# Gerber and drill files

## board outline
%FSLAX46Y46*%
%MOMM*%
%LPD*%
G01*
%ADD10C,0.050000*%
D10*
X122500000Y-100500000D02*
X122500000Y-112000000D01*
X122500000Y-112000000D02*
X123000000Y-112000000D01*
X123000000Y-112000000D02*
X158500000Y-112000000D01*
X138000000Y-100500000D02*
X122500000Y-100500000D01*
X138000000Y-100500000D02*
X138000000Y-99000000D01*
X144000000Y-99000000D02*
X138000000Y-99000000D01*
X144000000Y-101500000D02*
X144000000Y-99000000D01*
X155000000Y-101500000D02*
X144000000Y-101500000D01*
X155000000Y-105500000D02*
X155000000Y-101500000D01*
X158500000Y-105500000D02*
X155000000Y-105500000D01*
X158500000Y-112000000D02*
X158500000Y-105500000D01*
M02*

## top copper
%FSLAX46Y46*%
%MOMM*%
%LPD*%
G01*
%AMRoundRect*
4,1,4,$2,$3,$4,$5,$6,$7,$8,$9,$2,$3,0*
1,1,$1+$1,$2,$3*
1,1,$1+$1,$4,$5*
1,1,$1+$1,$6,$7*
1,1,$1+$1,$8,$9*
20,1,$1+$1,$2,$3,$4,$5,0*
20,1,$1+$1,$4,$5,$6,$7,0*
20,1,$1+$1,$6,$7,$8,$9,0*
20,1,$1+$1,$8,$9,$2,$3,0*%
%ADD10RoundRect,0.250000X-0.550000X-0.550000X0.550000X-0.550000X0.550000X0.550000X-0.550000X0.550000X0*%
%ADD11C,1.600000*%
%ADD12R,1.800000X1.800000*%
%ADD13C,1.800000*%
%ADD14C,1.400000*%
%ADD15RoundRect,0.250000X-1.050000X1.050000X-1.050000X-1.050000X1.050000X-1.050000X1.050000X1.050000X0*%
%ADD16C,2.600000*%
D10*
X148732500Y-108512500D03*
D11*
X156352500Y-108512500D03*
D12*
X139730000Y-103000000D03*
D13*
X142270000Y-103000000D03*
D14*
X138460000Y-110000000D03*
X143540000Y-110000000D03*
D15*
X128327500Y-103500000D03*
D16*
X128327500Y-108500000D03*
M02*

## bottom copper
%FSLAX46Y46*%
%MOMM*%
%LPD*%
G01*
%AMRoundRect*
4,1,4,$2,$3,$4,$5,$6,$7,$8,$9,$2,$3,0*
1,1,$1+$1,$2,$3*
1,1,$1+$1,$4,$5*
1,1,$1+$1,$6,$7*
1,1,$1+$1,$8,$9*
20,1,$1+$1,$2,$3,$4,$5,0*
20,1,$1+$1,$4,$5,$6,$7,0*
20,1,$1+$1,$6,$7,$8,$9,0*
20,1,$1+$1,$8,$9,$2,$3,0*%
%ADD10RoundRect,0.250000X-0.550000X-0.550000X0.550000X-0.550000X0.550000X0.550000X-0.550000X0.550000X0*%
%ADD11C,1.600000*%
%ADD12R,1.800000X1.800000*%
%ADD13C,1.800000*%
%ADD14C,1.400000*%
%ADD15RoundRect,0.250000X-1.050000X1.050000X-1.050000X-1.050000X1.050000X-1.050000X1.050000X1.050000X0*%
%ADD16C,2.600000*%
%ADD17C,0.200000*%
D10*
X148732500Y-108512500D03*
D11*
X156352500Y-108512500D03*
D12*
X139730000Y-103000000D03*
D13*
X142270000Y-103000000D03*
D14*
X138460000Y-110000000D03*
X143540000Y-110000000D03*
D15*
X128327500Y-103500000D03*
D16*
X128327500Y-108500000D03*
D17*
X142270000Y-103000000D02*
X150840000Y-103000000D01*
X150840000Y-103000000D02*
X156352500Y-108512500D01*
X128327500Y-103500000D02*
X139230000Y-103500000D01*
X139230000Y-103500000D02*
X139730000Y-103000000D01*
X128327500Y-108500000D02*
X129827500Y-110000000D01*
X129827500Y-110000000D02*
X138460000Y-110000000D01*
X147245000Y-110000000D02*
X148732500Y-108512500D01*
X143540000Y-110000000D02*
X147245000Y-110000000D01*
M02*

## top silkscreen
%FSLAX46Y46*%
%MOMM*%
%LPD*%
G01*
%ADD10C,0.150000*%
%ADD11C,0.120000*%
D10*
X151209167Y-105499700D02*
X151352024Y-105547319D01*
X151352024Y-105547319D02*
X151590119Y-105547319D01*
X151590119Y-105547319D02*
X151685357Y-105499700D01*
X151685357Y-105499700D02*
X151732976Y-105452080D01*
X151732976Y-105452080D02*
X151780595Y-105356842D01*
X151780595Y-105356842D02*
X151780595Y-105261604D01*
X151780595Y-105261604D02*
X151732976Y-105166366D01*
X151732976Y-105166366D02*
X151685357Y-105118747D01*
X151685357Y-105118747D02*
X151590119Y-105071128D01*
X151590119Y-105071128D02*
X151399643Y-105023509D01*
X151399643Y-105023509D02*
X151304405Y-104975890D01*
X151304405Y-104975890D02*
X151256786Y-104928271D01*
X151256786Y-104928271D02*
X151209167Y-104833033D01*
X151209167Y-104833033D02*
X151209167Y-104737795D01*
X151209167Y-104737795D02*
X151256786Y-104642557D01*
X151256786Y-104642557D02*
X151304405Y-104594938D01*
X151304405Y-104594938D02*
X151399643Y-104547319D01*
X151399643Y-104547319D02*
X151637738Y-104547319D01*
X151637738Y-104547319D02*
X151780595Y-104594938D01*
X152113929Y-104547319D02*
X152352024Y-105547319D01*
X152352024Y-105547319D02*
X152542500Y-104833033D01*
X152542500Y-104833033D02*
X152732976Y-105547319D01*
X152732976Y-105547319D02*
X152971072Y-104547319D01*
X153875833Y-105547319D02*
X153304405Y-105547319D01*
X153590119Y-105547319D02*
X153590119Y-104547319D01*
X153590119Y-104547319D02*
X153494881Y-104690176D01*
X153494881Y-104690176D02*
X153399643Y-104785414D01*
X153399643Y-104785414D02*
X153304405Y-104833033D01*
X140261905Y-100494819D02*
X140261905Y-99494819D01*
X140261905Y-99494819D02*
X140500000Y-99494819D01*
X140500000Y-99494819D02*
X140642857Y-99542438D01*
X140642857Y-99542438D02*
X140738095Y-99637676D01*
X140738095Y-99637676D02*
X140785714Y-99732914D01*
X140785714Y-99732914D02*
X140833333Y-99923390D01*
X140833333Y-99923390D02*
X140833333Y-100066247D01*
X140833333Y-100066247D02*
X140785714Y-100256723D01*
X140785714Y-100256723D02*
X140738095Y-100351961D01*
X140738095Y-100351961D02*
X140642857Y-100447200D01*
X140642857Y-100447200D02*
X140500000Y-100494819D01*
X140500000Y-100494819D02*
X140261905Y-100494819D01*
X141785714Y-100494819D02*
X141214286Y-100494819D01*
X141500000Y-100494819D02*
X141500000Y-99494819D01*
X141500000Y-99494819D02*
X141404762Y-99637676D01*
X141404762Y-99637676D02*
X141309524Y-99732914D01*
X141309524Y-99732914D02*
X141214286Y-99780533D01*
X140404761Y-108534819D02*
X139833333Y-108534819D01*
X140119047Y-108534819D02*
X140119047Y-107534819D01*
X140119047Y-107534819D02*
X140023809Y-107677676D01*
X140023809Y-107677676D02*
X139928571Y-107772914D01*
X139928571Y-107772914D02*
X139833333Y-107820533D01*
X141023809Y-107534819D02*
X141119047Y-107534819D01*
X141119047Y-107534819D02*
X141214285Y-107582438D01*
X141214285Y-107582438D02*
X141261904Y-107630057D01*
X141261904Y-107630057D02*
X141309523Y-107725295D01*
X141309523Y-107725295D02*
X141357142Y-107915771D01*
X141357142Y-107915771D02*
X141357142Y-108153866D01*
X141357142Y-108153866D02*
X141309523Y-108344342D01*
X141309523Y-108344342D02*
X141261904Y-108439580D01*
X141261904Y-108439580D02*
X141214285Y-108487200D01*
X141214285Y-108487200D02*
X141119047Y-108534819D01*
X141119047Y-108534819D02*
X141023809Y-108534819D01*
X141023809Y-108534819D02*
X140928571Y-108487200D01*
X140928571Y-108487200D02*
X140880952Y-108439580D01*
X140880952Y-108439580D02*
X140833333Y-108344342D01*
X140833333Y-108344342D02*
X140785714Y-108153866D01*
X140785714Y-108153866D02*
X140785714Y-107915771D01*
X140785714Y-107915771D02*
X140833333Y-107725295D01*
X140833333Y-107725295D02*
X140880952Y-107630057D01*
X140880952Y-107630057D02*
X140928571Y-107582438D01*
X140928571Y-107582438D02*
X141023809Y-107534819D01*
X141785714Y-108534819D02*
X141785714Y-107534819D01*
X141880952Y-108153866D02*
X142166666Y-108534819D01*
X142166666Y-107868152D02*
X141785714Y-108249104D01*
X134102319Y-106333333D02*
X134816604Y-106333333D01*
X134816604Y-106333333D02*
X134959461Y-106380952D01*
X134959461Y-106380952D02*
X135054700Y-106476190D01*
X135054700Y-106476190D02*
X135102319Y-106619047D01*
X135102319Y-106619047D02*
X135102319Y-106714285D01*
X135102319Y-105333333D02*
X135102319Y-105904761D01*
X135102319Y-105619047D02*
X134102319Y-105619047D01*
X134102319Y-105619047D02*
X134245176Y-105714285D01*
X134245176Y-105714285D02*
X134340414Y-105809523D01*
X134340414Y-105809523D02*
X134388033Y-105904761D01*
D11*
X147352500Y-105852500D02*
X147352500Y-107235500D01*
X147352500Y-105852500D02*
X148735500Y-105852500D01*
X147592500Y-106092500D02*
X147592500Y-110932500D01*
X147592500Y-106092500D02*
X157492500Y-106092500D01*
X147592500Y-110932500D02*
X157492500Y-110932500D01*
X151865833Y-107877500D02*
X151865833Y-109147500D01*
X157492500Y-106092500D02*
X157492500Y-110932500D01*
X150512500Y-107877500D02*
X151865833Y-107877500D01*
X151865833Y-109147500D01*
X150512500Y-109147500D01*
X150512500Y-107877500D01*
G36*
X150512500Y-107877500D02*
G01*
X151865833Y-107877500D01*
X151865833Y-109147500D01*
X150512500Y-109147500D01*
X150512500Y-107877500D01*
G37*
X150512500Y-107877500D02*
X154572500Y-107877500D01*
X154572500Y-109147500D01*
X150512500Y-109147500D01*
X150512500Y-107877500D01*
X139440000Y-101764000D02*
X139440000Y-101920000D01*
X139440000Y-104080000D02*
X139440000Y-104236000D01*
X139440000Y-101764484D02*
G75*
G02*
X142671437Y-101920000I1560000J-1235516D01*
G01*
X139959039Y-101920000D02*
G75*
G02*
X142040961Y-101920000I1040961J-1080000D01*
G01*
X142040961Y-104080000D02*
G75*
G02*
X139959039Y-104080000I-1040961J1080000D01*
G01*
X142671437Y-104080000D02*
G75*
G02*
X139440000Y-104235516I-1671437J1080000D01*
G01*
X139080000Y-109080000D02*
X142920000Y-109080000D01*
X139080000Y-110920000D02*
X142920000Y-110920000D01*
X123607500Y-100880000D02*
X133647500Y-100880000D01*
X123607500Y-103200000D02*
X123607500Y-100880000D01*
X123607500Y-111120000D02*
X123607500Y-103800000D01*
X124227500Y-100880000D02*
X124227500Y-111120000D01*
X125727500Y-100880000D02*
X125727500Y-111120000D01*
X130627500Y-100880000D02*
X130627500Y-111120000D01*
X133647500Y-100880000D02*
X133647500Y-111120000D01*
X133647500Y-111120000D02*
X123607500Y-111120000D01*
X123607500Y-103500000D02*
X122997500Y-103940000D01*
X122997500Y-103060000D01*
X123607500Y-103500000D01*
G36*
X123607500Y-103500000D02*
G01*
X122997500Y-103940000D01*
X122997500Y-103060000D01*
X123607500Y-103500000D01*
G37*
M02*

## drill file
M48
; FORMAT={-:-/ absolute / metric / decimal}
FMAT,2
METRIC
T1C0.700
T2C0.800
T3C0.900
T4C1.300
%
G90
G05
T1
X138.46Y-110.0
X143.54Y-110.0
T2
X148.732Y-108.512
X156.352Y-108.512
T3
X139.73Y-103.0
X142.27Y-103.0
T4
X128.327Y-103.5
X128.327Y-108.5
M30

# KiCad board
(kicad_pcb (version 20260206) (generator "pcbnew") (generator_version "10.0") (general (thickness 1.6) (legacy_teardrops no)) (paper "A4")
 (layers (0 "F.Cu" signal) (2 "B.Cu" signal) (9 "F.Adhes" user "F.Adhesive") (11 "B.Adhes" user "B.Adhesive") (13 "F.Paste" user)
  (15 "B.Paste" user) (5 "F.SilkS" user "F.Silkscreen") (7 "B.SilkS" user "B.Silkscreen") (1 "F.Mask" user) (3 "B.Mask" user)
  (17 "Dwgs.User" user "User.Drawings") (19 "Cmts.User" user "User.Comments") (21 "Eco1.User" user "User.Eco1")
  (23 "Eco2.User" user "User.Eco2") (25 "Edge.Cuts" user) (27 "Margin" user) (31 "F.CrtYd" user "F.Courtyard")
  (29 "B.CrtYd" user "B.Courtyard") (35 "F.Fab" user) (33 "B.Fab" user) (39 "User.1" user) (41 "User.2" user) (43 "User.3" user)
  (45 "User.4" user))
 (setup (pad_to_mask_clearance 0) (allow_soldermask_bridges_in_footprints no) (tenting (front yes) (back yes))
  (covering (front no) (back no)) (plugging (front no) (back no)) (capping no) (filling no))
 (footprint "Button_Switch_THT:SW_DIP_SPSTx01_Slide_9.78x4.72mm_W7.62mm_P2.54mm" (layer "F.Cu") (at 148.7325 108.5125)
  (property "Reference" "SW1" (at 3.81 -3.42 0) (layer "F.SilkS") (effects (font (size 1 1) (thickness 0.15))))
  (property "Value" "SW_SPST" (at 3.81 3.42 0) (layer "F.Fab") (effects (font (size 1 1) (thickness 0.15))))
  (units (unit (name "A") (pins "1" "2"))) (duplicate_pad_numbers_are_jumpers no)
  (fp_line (start -1.38 -2.66) (end -1.38 -1.277) (stroke (width 0.12) (type solid)) (layer "F.SilkS"))
  (fp_line (start -1.38 -2.66) (end 0.003 -2.66) (stroke (width 0.12) (type solid)) (layer "F.SilkS"))
  (fp_line (start -1.14 -2.42) (end -1.14 2.42) (stroke (width 0.12) (type solid)) (layer "F.SilkS"))
  (fp_line (start -1.14 -2.42) (end 8.76 -2.42) (stroke (width 0.12) (type solid)) (layer "F.SilkS"))
  (fp_line (start -1.14 2.42) (end 8.76 2.42) (stroke (width 0.12) (type solid)) (layer "F.SilkS"))
  (fp_line (start 3.133333 -0.635) (end 3.133333 0.635) (stroke (width 0.12) (type solid)) (layer "F.SilkS"))
  (fp_line (start 8.76 -2.42) (end 8.76 2.42) (stroke (width 0.12) (type solid)) (layer "F.SilkS"))
  (fp_rect (start 1.78 -0.635) (end 3.133333 0.635) (stroke (width 0.12) (type solid)) (fill yes) (layer "F.SilkS"))
  (fp_rect (start 1.78 -0.635) (end 5.84 0.635) (stroke (width 0.12) (type solid)) (fill no) (layer "F.SilkS"))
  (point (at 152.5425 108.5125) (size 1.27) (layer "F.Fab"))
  (pad "1" thru_hole roundrect (at 0 0) (size 1.6 1.6) (drill 0.8) (layers "*.Cu" "*.Mask") (remove_unused_layers no)
   (roundrect_rratio 0.15625) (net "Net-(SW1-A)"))
  (pad "2" thru_hole circle (at 7.62 0) (size 1.6 1.6) (drill 0.8) (layers "*.Cu" "*.Mask") (remove_unused_layers no) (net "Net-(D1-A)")))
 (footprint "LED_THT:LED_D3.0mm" (layer "F.Cu") (at 139.73 103)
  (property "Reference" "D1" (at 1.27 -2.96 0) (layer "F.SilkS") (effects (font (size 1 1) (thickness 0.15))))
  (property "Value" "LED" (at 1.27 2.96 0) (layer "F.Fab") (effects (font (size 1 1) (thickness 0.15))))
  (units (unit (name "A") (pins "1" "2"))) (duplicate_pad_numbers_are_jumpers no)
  (fp_line (start -0.29 -1.236) (end -0.29 -1.08) (stroke (width 0.12) (type solid)) (layer "F.SilkS"))
  (fp_line (start -0.29 1.08) (end -0.29 1.236) (stroke (width 0.12) (type solid)) (layer "F.SilkS"))
  (fp_arc (start -0.29 -1.235516) (mid 1.36566 -1.987699) (end 2.941437 -1.08) (stroke (width 0.12) (type solid)) (layer "F.SilkS"))
  (fp_arc (start 0.229039 -1.08) (mid 1.27 -1.5) (end 2.310961 -1.08) (stroke (width 0.12) (type solid)) (layer "F.SilkS"))
  (fp_arc (start 2.310961 1.08) (mid 1.27 1.5) (end 0.229039 1.08) (stroke (width 0.12) (type solid)) (layer "F.SilkS"))
  (fp_arc (start 2.941437 1.08) (mid 1.36566 1.987699) (end -0.29 1.235516) (stroke (width 0.12) (type solid)) (layer "F.SilkS"))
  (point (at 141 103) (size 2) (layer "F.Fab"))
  (pad "1" thru_hole rect (at 0 0) (size 1.8 1.8) (drill 0.9) (layers "*.Cu" "*.Mask") (remove_unused_layers no) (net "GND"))
  (pad "2" thru_hole circle (at 2.54 0) (size 1.8 1.8) (drill 0.9) (layers "*.Cu" "*.Mask") (remove_unused_layers no) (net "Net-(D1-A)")))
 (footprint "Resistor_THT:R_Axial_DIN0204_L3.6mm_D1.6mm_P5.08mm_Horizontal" (layer "F.Cu") (at 138.46 110)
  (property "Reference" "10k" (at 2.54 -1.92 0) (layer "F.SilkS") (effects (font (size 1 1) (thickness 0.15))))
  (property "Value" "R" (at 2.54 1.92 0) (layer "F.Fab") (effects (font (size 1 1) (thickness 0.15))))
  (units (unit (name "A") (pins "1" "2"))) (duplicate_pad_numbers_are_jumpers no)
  (fp_line (start 0.62 -0.92) (end 4.46 -0.92) (stroke (width 0.12) (type solid)) (layer "F.SilkS"))
  (fp_line (start 0.62 0.92) (end 4.46 0.92) (stroke (width 0.12) (type solid)) (layer "F.SilkS"))
  (pad "1" thru_hole circle (at 0 0) (size 1.4 1.4) (drill 0.7) (layers "*.Cu" "*.Mask") (remove_unused_layers no) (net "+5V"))
  (pad "2" thru_hole circle (at 5.08 0) (size 1.4 1.4) (drill 0.7) (layers "*.Cu" "*.Mask") (remove_unused_layers no) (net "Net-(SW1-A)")))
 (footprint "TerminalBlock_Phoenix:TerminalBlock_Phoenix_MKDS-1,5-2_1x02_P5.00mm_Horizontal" (layer "F.Cu") (at 128.3275 103.5 -90)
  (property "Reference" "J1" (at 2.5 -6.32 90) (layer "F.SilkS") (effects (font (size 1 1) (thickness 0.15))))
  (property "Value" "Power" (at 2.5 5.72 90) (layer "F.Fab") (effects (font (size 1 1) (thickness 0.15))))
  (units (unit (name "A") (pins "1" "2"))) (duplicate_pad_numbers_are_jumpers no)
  (fp_line (start -2.62 4.72) (end -2.62 -5.32) (stroke (width 0.12) (type solid)) (layer "F.SilkS"))
  (fp_line (start -0.3 4.72) (end -2.62 4.72) (stroke (width 0.12) (type solid)) (layer "F.SilkS"))
  (fp_line (start 7.62 4.72) (end 0.3 4.72) (stroke (width 0.12) (type solid)) (layer "F.SilkS"))
  (fp_line (start -2.62 4.1) (end 7.62 4.1) (stroke (width 0.12) (type solid)) (layer "F.SilkS"))
  (fp_line (start -2.62 2.6) (end 7.62 2.6) (stroke (width 0.12) (type solid)) (layer "F.SilkS"))
  (fp_line (start -2.62 -2.3) (end 7.62 -2.3) (stroke (width 0.12) (type solid)) (layer "F.SilkS"))
  (fp_line (start -2.62 -5.32) (end 7.62 -5.32) (stroke (width 0.12) (type solid)) (layer "F.SilkS"))
  (fp_line (start 7.62 -5.32) (end 7.62 4.72) (stroke (width 0.12) (type solid)) (layer "F.SilkS"))
  (fp_poly (pts (xy 0 4.72) (xy 0.44 5.33) (xy -0.44 5.33)) (stroke (width 0.12) (type solid)) (fill yes) (layer "F.SilkS"))
  (pad "1" thru_hole roundrect (at 0 0 270) (size 2.6 2.6) (drill 1.3) (layers "*.Cu" "*.Mask") (remove_unused_layers no)
   (roundrect_rratio 0.096154) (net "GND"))
  (pad "2" thru_hole circle (at 5 0 270) (size 2.6 2.6) (drill 1.3) (layers "*.Cu" "*.Mask") (remove_unused_layers no) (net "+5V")))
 (gr_line (start 122.5 100.5) (end 122.5 112) (stroke (width 0.05) (type default)) (layer "Edge.Cuts"))
 (gr_line (start 122.5 112) (end 123 112) (stroke (width 0.05) (type default)) (layer "Edge.Cuts"))
 (gr_line (start 123 112) (end 158.5 112) (stroke (width 0.05) (type default)) (layer "Edge.Cuts"))
 (gr_line (start 138 100.5) (end 122.5 100.5) (stroke (width 0.05) (type default)) (layer "Edge.Cuts"))
 (gr_line (start 138 100.5) (end 138 99) (stroke (width 0.05) (type default)) (layer "Edge.Cuts"))
 (gr_line (start 144 99) (end 138 99) (stroke (width 0.05) (type default)) (layer "Edge.Cuts"))
 (gr_line (start 144 101.5) (end 144 99) (stroke (width 0.05) (type default)) (layer "Edge.Cuts"))
 (gr_line (start 155 101.5) (end 144 101.5) (stroke (width 0.05) (type default)) (layer "Edge.Cuts"))
 (gr_line (start 155 105.5) (end 155 101.5) (stroke (width 0.05) (type default)) (layer "Edge.Cuts"))
 (gr_line (start 158.5 105.5) (end 155 105.5) (stroke (width 0.05) (type default)) (layer "Edge.Cuts"))
 (gr_line (start 158.5 112) (end 158.5 105.5) (stroke (width 0.05) (type default)) (layer "Edge.Cuts"))
 (segment (start 142.27 103) (end 150.84 103) (width 0.2) (layer "B.Cu") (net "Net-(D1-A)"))
 (segment (start 150.84 103) (end 156.3525 108.5125) (width 0.2) (layer "B.Cu") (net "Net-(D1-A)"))
 (segment (start 128.3275 103.5) (end 139.23 103.5) (width 0.2) (layer "B.Cu") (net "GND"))
 (segment (start 139.23 103.5) (end 139.73 103) (width 0.2) (layer "B.Cu") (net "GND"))
 (segment (start 128.3275 108.5) (end 129.8275 110) (width 0.2) (layer "B.Cu") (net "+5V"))
 (segment (start 129.8275 110) (end 138.46 110) (width 0.2) (layer "B.Cu") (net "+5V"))
 (segment (start 147.245 110) (end 148.7325 108.5125) (width 0.2) (layer "B.Cu") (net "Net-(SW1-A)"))
 (segment (start 143.54 110) (end 147.245 110) (width 0.2) (layer "B.Cu") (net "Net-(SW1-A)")))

